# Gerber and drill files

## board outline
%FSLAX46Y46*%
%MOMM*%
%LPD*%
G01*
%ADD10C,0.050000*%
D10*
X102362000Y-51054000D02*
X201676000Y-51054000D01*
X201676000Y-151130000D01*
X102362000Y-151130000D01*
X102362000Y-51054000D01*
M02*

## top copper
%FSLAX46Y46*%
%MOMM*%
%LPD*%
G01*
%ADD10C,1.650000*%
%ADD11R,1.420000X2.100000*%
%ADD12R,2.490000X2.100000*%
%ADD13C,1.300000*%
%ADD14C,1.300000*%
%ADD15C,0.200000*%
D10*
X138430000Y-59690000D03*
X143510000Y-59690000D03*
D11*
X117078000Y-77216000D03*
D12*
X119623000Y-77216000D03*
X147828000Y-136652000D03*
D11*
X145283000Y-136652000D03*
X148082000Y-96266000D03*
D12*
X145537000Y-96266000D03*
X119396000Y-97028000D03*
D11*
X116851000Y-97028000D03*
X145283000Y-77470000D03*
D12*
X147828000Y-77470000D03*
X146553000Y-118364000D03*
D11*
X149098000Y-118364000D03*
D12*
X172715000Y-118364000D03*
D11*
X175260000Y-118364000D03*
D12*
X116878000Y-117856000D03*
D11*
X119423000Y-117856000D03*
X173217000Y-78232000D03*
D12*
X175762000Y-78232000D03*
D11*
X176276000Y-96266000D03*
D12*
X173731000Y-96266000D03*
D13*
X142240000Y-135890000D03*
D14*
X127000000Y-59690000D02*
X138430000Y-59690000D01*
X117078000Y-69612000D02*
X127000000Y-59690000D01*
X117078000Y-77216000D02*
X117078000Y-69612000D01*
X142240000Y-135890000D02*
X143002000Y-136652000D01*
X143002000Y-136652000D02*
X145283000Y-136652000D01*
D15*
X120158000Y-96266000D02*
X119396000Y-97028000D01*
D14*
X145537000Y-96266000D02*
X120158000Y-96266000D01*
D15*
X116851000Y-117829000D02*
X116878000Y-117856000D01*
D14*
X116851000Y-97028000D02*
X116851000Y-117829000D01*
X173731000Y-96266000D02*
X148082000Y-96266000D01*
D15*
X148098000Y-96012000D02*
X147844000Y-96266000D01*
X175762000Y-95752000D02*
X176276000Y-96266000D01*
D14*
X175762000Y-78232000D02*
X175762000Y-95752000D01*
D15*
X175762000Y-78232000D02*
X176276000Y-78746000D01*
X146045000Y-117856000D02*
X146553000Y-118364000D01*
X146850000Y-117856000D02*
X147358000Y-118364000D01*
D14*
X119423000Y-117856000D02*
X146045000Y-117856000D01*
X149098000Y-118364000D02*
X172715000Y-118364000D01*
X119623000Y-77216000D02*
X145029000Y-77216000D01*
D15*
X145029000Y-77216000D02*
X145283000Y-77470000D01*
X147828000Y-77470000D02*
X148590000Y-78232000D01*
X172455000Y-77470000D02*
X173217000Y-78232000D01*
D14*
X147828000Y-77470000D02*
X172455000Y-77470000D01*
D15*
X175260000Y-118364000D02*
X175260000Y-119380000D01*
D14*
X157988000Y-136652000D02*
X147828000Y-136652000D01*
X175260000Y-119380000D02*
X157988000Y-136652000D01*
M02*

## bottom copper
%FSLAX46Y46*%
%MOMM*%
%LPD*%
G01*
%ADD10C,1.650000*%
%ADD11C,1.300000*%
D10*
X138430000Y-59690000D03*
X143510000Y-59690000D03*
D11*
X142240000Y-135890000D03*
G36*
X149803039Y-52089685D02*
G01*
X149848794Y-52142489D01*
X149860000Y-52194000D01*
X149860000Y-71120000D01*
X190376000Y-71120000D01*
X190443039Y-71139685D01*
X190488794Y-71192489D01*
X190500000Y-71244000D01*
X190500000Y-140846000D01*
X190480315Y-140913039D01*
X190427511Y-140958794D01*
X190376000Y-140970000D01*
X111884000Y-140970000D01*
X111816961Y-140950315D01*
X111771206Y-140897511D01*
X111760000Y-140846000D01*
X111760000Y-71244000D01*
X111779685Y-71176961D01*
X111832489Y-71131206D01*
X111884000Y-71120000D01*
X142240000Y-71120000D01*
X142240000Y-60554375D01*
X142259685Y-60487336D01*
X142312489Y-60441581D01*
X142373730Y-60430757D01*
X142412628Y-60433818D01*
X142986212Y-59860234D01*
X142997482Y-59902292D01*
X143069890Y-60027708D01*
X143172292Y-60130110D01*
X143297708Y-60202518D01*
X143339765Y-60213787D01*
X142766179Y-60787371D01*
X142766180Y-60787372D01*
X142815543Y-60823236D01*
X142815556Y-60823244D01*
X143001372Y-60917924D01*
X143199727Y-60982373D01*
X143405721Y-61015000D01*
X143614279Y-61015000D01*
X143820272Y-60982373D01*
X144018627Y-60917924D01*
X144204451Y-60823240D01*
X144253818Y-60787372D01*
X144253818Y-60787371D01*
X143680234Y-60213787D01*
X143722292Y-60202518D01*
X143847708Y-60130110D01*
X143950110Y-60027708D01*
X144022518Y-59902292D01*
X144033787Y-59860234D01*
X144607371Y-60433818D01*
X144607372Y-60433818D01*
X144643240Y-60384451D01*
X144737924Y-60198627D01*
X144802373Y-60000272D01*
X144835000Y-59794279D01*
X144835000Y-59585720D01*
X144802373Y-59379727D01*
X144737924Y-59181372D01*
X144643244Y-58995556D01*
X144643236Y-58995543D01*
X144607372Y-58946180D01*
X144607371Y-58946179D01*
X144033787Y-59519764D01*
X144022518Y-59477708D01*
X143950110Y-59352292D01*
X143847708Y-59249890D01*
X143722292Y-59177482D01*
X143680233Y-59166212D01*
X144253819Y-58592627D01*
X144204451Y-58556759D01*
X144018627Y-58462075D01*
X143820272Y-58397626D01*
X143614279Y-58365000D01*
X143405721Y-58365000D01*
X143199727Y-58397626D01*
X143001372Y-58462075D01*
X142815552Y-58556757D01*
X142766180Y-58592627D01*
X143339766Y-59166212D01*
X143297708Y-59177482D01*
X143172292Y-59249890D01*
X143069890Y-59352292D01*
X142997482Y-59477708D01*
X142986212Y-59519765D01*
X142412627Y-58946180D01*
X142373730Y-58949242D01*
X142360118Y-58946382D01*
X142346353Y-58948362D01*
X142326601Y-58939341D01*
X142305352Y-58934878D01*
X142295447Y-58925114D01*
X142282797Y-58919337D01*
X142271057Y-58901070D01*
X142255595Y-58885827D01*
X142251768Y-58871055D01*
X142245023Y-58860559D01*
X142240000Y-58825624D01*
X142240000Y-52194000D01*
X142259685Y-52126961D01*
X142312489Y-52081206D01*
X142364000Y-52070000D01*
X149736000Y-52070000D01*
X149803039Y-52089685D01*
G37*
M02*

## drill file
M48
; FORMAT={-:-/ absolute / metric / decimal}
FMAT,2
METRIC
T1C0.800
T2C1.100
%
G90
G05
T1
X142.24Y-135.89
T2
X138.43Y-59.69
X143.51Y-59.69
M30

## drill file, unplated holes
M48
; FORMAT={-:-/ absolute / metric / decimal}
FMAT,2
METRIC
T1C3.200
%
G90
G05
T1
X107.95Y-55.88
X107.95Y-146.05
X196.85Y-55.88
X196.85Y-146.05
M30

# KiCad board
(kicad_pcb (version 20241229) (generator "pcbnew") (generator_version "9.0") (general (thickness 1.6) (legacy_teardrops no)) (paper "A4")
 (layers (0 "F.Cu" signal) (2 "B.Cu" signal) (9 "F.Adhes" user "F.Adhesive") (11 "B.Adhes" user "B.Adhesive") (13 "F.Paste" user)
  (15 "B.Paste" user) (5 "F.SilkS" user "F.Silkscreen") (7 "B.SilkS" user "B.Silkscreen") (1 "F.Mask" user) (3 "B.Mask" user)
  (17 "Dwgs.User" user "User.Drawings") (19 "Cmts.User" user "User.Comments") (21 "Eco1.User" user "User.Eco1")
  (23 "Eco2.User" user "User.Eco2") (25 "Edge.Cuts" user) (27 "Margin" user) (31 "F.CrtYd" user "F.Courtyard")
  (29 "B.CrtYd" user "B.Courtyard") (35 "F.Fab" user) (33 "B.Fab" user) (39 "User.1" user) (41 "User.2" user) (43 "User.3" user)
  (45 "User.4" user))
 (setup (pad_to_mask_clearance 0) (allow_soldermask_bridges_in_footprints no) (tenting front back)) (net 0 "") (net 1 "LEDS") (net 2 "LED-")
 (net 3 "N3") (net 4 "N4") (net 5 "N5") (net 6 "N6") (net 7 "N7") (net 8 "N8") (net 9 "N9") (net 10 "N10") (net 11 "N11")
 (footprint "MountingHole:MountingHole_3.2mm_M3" (layer "F.Cu") (at 107.95 146.05)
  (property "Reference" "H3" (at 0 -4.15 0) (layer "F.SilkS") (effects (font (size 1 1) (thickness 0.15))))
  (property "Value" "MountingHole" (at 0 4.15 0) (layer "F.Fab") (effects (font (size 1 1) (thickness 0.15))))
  (pad "" np_thru_hole circle (at 0 0) (size 3.2 3.2) (drill 3.2) (layers "*.Cu" "*.Mask")))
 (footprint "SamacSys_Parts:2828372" (layer "F.Cu") (at 138.43 59.69)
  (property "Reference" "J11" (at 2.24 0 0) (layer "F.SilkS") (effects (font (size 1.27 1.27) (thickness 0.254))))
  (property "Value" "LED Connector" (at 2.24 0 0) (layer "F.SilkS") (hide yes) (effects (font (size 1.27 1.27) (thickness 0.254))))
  (pad "1" thru_hole circle (at 0 0) (size 1.65 1.65) (drill 1.1) (layers "*.Cu" "*.Mask") (remove_unused_layers no) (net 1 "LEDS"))
  (pad "2" thru_hole circle (at 5.08 0) (size 1.65 1.65) (drill 1.1) (layers "*.Cu" "*.Mask") (remove_unused_layers no) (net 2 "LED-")))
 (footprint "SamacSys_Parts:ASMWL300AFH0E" (layer "F.Cu") (at 118.618 77.216 180)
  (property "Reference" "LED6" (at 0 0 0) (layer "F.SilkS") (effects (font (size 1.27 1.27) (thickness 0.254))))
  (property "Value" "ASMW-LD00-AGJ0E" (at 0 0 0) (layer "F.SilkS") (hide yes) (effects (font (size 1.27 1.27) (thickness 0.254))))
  (pad "1" smd rect (at 1.54 0 180) (size 1.42 2.1) (layers "F.Cu" "F.Mask" "F.Paste") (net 1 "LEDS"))
  (pad "2" smd rect (at -1.005 0 270) (size 2.1 2.49) (layers "F.Cu" "F.Mask" "F.Paste") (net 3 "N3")))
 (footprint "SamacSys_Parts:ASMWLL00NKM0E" (layer "F.Cu") (at 146.823 136.652)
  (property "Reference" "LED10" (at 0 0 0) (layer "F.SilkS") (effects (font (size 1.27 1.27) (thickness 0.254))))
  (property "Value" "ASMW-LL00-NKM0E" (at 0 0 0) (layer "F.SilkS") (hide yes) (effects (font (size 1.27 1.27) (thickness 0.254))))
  (pad "1" smd rect (at 1.005 0 90) (size 2.1 2.49) (layers "F.Cu" "F.Mask" "F.Paste") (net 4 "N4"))
  (pad "2" smd rect (at -1.54 0) (size 1.42 2.1) (layers "F.Cu" "F.Mask" "F.Paste") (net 2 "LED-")))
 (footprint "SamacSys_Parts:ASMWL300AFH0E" (layer "F.Cu") (at 146.542 96.266)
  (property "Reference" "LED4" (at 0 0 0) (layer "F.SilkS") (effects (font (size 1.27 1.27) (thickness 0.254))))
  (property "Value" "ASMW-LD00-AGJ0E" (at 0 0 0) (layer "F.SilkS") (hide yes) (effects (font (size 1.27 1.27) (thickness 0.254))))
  (pad "1" smd rect (at 1.54 0) (size 1.42 2.1) (layers "F.Cu" "F.Mask" "F.Paste") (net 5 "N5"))
  (pad "2" smd rect (at -1.005 0 90) (size 2.1 2.49) (layers "F.Cu" "F.Mask" "F.Paste") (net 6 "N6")))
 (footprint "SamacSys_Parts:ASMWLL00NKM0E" (layer "F.Cu") (at 118.391 97.028)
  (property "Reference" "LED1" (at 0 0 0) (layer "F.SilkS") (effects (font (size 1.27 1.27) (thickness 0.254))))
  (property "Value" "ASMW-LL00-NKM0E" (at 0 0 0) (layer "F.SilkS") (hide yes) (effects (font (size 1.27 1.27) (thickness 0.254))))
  (pad "1" smd rect (at 1.005 0 90) (size 2.1 2.49) (layers "F.Cu" "F.Mask" "F.Paste") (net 6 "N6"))
  (pad "2" smd rect (at -1.54 0) (size 1.42 2.1) (layers "F.Cu" "F.Mask" "F.Paste") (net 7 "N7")))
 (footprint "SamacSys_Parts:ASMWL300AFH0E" (layer "F.Cu") (at 146.823 77.47 180)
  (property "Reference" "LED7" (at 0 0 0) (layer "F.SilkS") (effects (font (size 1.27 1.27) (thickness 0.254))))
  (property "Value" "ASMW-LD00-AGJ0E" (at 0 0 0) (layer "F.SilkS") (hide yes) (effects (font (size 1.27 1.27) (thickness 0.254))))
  (pad "1" smd rect (at 1.54 0 180) (size 1.42 2.1) (layers "F.Cu" "F.Mask" "F.Paste") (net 3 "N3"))
  (pad "2" smd rect (at -1.005 0 270) (size 2.1 2.49) (layers "F.Cu" "F.Mask" "F.Paste") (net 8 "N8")))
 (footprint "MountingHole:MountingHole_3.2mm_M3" (layer "F.Cu") (at 107.95 55.88)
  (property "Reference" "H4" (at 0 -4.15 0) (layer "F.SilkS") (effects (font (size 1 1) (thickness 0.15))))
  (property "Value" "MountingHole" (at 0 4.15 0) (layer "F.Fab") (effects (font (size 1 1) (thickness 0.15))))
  (pad "" np_thru_hole circle (at 0 0) (size 3.2 3.2) (drill 3.2) (layers "*.Cu" "*.Mask")))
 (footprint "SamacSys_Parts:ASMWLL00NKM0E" (layer "F.Cu") (at 147.558 118.364 180)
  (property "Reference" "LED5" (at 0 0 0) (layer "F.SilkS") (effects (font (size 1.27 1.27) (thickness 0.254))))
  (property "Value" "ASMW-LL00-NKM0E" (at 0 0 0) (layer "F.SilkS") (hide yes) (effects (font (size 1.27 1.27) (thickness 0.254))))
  (pad "1" smd rect (at 1.005 0 270) (size 2.1 2.49) (layers "F.Cu" "F.Mask" "F.Paste") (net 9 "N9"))
  (pad "2" smd rect (at -1.54 0 180) (size 1.42 2.1) (layers "F.Cu" "F.Mask" "F.Paste") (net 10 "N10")))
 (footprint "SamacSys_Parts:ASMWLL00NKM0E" (layer "F.Cu") (at 173.72 118.364 180)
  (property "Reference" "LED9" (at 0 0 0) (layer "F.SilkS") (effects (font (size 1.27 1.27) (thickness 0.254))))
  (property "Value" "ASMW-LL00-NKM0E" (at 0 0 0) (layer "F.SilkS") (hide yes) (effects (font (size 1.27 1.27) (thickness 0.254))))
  (pad "1" smd rect (at 1.005 0 270) (size 2.1 2.49) (layers "F.Cu" "F.Mask" "F.Paste") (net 10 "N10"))
  (pad "2" smd rect (at -1.54 0 180) (size 1.42 2.1) (layers "F.Cu" "F.Mask" "F.Paste") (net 4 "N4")))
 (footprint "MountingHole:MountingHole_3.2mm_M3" (layer "F.Cu") (at 196.85 146.05)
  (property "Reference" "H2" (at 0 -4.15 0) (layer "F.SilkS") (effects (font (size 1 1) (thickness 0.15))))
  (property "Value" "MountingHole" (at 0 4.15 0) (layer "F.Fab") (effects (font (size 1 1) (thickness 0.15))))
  (pad "" np_thru_hole circle (at 0 0) (size 3.2 3.2) (drill 3.2) (layers "*.Cu" "*.Mask")))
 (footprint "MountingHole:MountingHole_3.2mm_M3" (layer "F.Cu") (at 196.85 55.88)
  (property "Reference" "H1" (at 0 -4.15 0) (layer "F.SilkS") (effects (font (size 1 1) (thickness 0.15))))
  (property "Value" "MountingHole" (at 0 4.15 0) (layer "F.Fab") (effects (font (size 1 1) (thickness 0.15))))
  (pad "" np_thru_hole circle (at 0 0) (size 3.2 3.2) (drill 3.2) (layers "*.Cu" "*.Mask")))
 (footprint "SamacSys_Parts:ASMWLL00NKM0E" (layer "F.Cu") (at 117.883 117.856 180)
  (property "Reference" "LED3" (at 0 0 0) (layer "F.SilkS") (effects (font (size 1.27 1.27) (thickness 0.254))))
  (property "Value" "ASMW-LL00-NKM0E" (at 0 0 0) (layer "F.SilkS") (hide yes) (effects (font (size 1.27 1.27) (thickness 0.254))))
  (pad "1" smd rect (at 1.005 0 270) (size 2.1 2.49) (layers "F.Cu" "F.Mask" "F.Paste") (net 7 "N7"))
  (pad "2" smd rect (at -1.54 0 180) (size 1.42 2.1) (layers "F.Cu" "F.Mask" "F.Paste") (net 9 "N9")))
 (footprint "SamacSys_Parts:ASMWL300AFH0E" (layer "F.Cu") (at 174.757 78.232 180)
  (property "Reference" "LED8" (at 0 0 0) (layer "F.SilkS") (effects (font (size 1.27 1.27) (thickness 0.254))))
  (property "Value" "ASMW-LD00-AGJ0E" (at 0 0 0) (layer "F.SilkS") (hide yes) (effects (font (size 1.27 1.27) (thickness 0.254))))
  (pad "1" smd rect (at 1.54 0 180) (size 1.42 2.1) (layers "F.Cu" "F.Mask" "F.Paste") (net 8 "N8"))
  (pad "2" smd rect (at -1.005 0 270) (size 2.1 2.49) (layers "F.Cu" "F.Mask" "F.Paste") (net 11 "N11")))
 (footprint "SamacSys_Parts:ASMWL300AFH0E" (layer "F.Cu") (at 174.736 96.266)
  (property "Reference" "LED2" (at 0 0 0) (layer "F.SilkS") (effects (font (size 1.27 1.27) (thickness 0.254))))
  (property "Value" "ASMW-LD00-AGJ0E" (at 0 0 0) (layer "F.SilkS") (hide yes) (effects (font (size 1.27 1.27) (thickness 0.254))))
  (pad "1" smd rect (at 1.54 0) (size 1.42 2.1) (layers "F.Cu" "F.Mask" "F.Paste") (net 11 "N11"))
  (pad "2" smd rect (at -1.005 0 90) (size 2.1 2.49) (layers "F.Cu" "F.Mask" "F.Paste") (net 5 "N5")))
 (gr_rect (start 102.362 51.054) (end 201.676 151.13) (stroke (width 0.05) (type default)) (fill no) (layer "Edge.Cuts"))
 (segment (start 142.24 135.89) (end 143.002 136.652) (width 1.3) (layer "F.Cu") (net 2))
 (segment (start 143.002 136.652) (end 145.283 136.652) (width 1.3) (layer "F.Cu") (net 2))
 (via (at 142.24 135.89) (size 1.3) (drill 0.8) (layers "F.Cu" "B.Cu") (free yes) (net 2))
 (segment (start 127 59.69) (end 138.43 59.69) (width 1.3) (layer "F.Cu") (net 1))
 (segment (start 117.078 77.216) (end 117.078 69.612) (width 1.3) (layer "F.Cu") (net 1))
 (segment (start 117.078 69.612) (end 127 59.69) (width 1.3) (layer "F.Cu") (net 1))
 (segment (start 120.158 96.266) (end 119.396 97.028) (width 0.2) (layer "F.Cu") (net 6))
 (segment (start 145.537 96.266) (end 120.158 96.266) (width 1.3) (layer "F.Cu") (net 6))
 (segment (start 116.851 117.829) (end 116.878 117.856) (width 0.2) (layer "F.Cu") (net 7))
 (segment (start 116.851 97.028) (end 116.851 117.829) (width 1.3) (layer "F.Cu") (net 7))
 (segment (start 173.731 96.266) (end 148.082 96.266) (width 1.3) (layer "F.Cu") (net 5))
 (segment (start 148.098 96.012) (end 147.844 96.266) (width 0.2) (layer "F.Cu") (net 5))
 (segment (start 175.762 95.752) (end 176.276 96.266) (width 0.2) (layer "F.Cu") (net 11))
 (segment (start 175.762 78.232) (end 175.762 95.752) (width 1.3) (layer "F.Cu") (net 11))
 (segment (start 175.762 78.232) (end 176.276 78.746) (width 0.2) (layer "F.Cu") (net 11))
 (segment (start 146.045 117.856) (end 146.553 118.364) (width 0.2) (layer "F.Cu") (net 9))
 (segment (start 146.85 117.856) (end 147.358 118.364) (width 0.2) (layer "F.Cu") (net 9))
 (segment (start 119.423 117.856) (end 146.045 117.856) (width 1.3) (layer "F.Cu") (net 9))
 (segment (start 149.098 118.364) (end 172.715 118.364) (width 1.3) (layer "F.Cu") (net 10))
 (segment (start 119.623 77.216) (end 145.029 77.216) (width 1.3) (layer "F.Cu") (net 3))
 (segment (start 145.029 77.216) (end 145.283 77.47) (width 0.2) (layer "F.Cu") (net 3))
 (segment (start 147.828 77.47) (end 148.59 78.232) (width 0.2) (layer "F.Cu") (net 8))
 (segment (start 172.455 77.47) (end 173.217 78.232) (width 0.2) (layer "F.Cu") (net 8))
 (segment (start 147.828 77.47) (end 172.455 77.47) (width 1.3) (layer "F.Cu") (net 8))
 (segment (start 175.26 118.364) (end 175.26 119.38) (width 0.2) (layer "F.Cu") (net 4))
 (segment (start 157.988 136.652) (end 147.828 136.652) (width 1.3) (layer "F.Cu") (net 4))
 (segment (start 175.26 119.38) (end 157.988 136.652) (width 1.3) (layer "F.Cu") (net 4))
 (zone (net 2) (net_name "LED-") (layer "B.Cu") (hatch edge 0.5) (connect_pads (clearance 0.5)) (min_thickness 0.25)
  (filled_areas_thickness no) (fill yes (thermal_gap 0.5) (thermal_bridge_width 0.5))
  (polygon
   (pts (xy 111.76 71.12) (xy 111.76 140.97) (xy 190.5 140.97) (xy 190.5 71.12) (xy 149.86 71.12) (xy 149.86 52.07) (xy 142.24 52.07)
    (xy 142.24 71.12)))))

